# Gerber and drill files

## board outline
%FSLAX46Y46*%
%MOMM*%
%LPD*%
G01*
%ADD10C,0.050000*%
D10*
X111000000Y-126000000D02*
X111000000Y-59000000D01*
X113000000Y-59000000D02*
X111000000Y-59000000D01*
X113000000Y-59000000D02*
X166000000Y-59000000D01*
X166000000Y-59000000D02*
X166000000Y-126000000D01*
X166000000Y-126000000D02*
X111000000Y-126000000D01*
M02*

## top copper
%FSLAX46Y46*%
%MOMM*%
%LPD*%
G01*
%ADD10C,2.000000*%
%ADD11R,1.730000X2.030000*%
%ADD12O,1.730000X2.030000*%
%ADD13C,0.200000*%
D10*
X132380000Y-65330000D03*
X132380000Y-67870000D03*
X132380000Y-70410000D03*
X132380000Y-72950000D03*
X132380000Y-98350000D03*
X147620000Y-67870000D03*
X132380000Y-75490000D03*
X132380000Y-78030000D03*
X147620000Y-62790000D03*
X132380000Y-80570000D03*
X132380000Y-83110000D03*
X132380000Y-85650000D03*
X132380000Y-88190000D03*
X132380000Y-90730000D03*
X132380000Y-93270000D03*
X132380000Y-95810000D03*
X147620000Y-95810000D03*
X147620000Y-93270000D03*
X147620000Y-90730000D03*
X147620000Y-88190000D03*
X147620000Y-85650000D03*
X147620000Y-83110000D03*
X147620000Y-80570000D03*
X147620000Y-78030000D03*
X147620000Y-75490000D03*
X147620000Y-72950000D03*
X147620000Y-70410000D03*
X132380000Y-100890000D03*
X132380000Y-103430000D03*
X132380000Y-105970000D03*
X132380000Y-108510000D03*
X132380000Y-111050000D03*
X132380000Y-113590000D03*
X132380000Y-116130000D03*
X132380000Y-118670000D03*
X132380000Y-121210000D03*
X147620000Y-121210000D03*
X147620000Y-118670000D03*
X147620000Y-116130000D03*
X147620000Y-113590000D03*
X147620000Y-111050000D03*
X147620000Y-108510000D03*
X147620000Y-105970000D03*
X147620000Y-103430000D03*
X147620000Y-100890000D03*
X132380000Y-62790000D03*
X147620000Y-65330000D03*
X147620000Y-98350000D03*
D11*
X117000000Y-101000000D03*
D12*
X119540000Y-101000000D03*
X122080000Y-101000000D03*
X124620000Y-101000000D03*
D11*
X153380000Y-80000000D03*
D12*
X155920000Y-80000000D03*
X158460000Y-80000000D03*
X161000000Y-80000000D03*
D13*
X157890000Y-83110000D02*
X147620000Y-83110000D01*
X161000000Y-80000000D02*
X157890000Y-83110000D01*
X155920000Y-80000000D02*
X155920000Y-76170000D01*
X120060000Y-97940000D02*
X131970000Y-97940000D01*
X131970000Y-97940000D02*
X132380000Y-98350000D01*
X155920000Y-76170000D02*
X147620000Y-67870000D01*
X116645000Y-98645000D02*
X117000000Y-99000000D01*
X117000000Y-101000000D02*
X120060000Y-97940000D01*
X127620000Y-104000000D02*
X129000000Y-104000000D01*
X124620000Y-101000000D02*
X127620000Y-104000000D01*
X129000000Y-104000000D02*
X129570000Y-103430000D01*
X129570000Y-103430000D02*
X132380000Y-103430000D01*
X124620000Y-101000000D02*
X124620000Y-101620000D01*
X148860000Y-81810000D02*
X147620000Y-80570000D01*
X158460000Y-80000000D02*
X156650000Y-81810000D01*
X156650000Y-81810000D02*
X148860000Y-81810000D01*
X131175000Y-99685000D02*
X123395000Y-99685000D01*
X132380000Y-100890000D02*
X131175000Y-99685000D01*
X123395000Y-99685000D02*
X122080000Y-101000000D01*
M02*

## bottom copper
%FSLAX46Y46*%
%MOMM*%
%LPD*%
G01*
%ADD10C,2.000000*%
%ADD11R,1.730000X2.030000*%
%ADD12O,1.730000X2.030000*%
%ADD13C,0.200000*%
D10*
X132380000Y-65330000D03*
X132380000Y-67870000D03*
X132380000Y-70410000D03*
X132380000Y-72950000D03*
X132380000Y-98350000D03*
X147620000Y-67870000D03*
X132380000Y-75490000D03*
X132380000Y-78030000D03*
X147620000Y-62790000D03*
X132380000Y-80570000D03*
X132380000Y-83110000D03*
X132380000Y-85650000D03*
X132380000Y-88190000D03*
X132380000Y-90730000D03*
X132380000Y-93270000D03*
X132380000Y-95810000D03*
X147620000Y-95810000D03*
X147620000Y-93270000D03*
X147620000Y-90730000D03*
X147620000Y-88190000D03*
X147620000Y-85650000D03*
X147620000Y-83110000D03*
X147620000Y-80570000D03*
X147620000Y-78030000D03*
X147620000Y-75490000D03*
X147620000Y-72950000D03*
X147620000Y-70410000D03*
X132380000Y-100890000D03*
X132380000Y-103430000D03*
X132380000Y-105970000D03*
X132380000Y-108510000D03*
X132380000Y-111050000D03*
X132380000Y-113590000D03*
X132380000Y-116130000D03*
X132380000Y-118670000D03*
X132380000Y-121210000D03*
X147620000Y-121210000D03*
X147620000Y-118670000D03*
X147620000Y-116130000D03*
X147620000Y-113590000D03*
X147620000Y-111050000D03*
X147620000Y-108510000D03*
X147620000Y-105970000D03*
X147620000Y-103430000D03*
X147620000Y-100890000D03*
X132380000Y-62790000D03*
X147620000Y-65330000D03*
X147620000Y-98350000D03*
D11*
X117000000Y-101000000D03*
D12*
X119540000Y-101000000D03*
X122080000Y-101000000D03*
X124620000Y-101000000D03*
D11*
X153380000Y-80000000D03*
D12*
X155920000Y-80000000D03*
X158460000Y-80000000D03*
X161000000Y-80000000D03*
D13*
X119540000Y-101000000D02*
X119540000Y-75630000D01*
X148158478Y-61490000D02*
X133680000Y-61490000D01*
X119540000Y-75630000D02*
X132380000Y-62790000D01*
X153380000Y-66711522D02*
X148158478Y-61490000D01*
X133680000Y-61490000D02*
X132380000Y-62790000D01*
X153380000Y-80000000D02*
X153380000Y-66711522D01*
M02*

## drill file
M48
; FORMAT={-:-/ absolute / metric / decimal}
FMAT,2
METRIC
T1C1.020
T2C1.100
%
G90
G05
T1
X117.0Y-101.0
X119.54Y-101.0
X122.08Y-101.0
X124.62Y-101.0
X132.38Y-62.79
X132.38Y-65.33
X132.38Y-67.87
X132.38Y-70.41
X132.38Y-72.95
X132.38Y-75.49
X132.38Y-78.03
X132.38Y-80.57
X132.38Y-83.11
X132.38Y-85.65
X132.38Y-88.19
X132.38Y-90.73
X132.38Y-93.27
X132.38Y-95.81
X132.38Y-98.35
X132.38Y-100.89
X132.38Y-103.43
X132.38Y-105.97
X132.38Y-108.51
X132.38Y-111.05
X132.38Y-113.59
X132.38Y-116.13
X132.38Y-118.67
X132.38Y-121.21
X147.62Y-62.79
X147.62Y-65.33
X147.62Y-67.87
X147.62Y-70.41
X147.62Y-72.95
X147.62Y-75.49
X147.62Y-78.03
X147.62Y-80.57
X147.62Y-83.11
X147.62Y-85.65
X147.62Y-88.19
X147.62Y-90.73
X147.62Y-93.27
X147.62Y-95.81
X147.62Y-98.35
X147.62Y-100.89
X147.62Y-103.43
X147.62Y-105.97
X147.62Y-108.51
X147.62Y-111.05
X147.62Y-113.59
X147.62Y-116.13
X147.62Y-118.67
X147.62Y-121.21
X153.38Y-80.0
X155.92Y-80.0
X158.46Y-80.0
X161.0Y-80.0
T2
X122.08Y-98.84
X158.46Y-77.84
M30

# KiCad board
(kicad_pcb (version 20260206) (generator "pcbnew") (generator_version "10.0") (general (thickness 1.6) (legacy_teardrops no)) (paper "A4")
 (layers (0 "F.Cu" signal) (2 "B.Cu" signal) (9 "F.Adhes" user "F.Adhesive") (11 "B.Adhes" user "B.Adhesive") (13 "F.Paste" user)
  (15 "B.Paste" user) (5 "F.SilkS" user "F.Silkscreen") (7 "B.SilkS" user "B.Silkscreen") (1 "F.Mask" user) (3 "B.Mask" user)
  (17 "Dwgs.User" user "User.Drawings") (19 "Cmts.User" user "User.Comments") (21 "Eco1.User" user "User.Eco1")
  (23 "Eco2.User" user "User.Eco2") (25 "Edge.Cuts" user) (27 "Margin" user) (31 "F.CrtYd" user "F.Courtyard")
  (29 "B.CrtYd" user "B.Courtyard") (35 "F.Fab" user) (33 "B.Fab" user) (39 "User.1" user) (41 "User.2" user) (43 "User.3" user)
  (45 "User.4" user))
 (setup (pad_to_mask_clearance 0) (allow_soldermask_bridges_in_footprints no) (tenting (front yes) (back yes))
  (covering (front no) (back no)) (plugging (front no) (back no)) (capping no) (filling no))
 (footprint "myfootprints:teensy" (layer "F.Cu") (at 140 92)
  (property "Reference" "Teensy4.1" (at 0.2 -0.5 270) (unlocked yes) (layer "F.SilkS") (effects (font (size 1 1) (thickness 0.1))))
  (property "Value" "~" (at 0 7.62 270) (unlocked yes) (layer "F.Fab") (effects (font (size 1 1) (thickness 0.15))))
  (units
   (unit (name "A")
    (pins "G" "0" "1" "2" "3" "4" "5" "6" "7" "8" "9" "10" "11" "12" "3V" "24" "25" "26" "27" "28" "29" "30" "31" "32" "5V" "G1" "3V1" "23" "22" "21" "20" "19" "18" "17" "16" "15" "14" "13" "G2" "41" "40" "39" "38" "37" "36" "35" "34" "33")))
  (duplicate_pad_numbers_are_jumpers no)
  (pad "0" thru_hole circle (at -7.62 -26.67) (size 2 2) (drill 1.02) (layers "*.Cu" "*.Mask") (remove_unused_layers no)
   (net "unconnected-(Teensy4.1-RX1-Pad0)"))
  (pad "1" thru_hole circle (at -7.62 -24.13) (size 2 2) (drill 1.02) (layers "*.Cu" "*.Mask") (remove_unused_layers no)
   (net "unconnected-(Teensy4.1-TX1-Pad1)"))
  (pad "2" thru_hole circle (at -7.62 -21.59) (size 2 2) (drill 1.02) (layers "*.Cu" "*.Mask") (remove_unused_layers no)
   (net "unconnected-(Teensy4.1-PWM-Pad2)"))
  (pad "3" thru_hole circle (at -7.62 -19.05) (size 2 2) (drill 1.02) (layers "*.Cu" "*.Mask") (remove_unused_layers no)
   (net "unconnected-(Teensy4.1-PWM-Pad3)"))
  (pad "3V" thru_hole circle (at -7.62 6.35) (size 2 2) (drill 1.02) (layers "*.Cu" "*.Mask") (remove_unused_layers no) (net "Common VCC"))
  (pad "3V1" thru_hole circle (at 7.62 -24.13) (size 2 2) (drill 1.02) (layers "*.Cu" "*.Mask") (remove_unused_layers no) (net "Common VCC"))
  (pad "4" thru_hole circle (at -7.62 -16.51) (size 2 2) (drill 1.02) (layers "*.Cu" "*.Mask") (remove_unused_layers no)
   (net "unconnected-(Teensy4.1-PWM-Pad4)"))
  (pad "5" thru_hole circle (at -7.62 -13.97) (size 2 2) (drill 1.02) (layers "*.Cu" "*.Mask") (remove_unused_layers no)
   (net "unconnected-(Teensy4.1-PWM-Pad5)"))
  (pad "5V" thru_hole circle (at 7.62 -29.21) (size 2 2) (drill 1.02) (layers "*.Cu" "*.Mask") (remove_unused_layers no) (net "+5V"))
  (pad "6" thru_hole circle (at -7.62 -11.43) (size 2 2) (drill 1.02) (layers "*.Cu" "*.Mask") (remove_unused_layers no)
   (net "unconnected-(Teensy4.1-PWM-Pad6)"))
  (pad "7" thru_hole circle (at -7.62 -8.89) (size 2 2) (drill 1.02) (layers "*.Cu" "*.Mask") (remove_unused_layers no)
   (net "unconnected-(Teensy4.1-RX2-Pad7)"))
  (pad "8" thru_hole circle (at -7.62 -6.35) (size 2 2) (drill 1.02) (layers "*.Cu" "*.Mask") (remove_unused_layers no)
   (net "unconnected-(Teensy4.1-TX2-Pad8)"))
  (pad "9" thru_hole circle (at -7.62 -3.81) (size 2 2) (drill 1.02) (layers "*.Cu" "*.Mask") (remove_unused_layers no)
   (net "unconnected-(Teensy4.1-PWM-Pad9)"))
  (pad "10" thru_hole circle (at -7.62 -1.27) (size 2 2) (drill 1.02) (layers "*.Cu" "*.Mask") (remove_unused_layers no)
   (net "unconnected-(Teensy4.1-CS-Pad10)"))
  (pad "11" thru_hole circle (at -7.62 1.27) (size 2 2) (drill 1.02) (layers "*.Cu" "*.Mask") (remove_unused_layers no)
   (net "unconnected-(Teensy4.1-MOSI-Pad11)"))
  (pad "12" thru_hole circle (at -7.62 3.81) (size 2 2) (drill 1.02) (layers "*.Cu" "*.Mask") (remove_unused_layers no)
   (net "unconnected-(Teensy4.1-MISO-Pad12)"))
  (pad "13" thru_hole circle (at 7.62 3.81) (size 2 2) (drill 1.02) (layers "*.Cu" "*.Mask") (remove_unused_layers no)
   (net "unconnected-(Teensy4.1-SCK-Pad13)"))
  (pad "14" thru_hole circle (at 7.62 1.27) (size 2 2) (drill 1.02) (layers "*.Cu" "*.Mask") (remove_unused_layers no)
   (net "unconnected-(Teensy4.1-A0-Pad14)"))
  (pad "15" thru_hole circle (at 7.62 -1.27) (size 2 2) (drill 1.02) (layers "*.Cu" "*.Mask") (remove_unused_layers no)
   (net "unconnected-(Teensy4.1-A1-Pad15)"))
  (pad "16" thru_hole circle (at 7.62 -3.81) (size 2 2) (drill 1.02) (layers "*.Cu" "*.Mask") (remove_unused_layers no)
   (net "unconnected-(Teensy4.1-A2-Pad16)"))
  (pad "17" thru_hole circle (at 7.62 -6.35) (size 2 2) (drill 1.02) (layers "*.Cu" "*.Mask") (remove_unused_layers no)
   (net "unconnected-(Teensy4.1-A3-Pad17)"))
  (pad "18" thru_hole circle (at 7.62 -8.89) (size 2 2) (drill 1.02) (layers "*.Cu" "*.Mask") (remove_unused_layers no) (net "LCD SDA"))
  (pad "19" thru_hole circle (at 7.62 -11.43) (size 2 2) (drill 1.02) (layers "*.Cu" "*.Mask") (remove_unused_layers no) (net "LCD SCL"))
  (pad "20" thru_hole circle (at 7.62 -13.97) (size 2 2) (drill 1.02) (layers "*.Cu" "*.Mask") (remove_unused_layers no)
   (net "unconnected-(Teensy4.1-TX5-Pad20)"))
  (pad "21" thru_hole circle (at 7.62 -16.51) (size 2 2) (drill 1.02) (layers "*.Cu" "*.Mask") (remove_unused_layers no)
   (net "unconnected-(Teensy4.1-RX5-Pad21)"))
  (pad "22" thru_hole circle (at 7.62 -19.05) (size 2 2) (drill 1.02) (layers "*.Cu" "*.Mask") (remove_unused_layers no)
   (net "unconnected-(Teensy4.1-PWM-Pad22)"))
  (pad "23" thru_hole circle (at 7.62 -21.59) (size 2 2) (drill 1.02) (layers "*.Cu" "*.Mask") (remove_unused_layers no)
   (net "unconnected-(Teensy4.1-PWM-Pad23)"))
  (pad "24" thru_hole circle (at -7.62 8.89) (size 2 2) (drill 1.02) (layers "*.Cu" "*.Mask") (remove_unused_layers no) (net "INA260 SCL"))
  (pad "25" thru_hole circle (at -7.62 11.43) (size 2 2) (drill 1.02) (layers "*.Cu" "*.Mask") (remove_unused_layers no) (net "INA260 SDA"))
  (pad "26" thru_hole circle (at -7.62 13.97) (size 2 2) (drill 1.02) (layers "*.Cu" "*.Mask") (remove_unused_layers no)
   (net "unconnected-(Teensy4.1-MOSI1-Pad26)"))
  (pad "27" thru_hole circle (at -7.62 16.51) (size 2 2) (drill 1.02) (layers "*.Cu" "*.Mask") (remove_unused_layers no)
   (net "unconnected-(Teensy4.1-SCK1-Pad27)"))
  (pad "28" thru_hole circle (at -7.62 19.05) (size 2 2) (drill 1.02) (layers "*.Cu" "*.Mask") (remove_unused_layers no)
   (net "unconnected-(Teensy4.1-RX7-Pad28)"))
  (pad "29" thru_hole circle (at -7.62 21.59) (size 2 2) (drill 1.02) (layers "*.Cu" "*.Mask") (remove_unused_layers no)
   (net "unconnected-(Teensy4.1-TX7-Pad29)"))
  (pad "30" thru_hole circle (at -7.62 24.13) (size 2 2) (drill 1.02) (layers "*.Cu" "*.Mask") (remove_unused_layers no)
   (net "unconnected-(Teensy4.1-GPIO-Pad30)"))
  (pad "31" thru_hole circle (at -7.62 26.67) (size 2 2) (drill 1.02) (layers "*.Cu" "*.Mask") (remove_unused_layers no)
   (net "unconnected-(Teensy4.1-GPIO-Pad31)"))
  (pad "32" thru_hole circle (at -7.62 29.21) (size 2 2) (drill 1.02) (layers "*.Cu" "*.Mask") (remove_unused_layers no)
   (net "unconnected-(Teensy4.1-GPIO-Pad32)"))
  (pad "33" thru_hole circle (at 7.62 29.21) (size 2 2) (drill 1.02) (layers "*.Cu" "*.Mask") (remove_unused_layers no)
   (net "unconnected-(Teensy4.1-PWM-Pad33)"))
  (pad "34" thru_hole circle (at 7.62 26.67) (size 2 2) (drill 1.02) (layers "*.Cu" "*.Mask") (remove_unused_layers no)
   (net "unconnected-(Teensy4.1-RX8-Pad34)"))
  (pad "35" thru_hole circle (at 7.62 24.13) (size 2 2) (drill 1.02) (layers "*.Cu" "*.Mask") (remove_unused_layers no)
   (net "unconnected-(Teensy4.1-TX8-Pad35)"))
  (pad "36" thru_hole circle (at 7.62 21.59) (size 2 2) (drill 1.02) (layers "*.Cu" "*.Mask") (remove_unused_layers no)
   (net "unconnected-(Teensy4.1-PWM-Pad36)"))
  (pad "37" thru_hole circle (at 7.62 19.05) (size 2 2) (drill 1.02) (layers "*.Cu" "*.Mask") (remove_unused_layers no)
   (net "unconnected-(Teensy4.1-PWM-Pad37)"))
  (pad "38" thru_hole circle (at 7.62 16.51) (size 2 2) (drill 1.02) (layers "*.Cu" "*.Mask") (remove_unused_layers no)
   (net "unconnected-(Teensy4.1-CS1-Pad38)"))
  (pad "39" thru_hole circle (at 7.62 13.97) (size 2 2) (drill 1.02) (layers "*.Cu" "*.Mask") (remove_unused_layers no)
   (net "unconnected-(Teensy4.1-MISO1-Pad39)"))
  (pad "40" thru_hole circle (at 7.62 11.43) (size 2 2) (drill 1.02) (layers "*.Cu" "*.Mask") (remove_unused_layers no)
   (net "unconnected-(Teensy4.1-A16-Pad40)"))
  (pad "41" thru_hole circle (at 7.62 8.89) (size 2 2) (drill 1.02) (layers "*.Cu" "*.Mask") (remove_unused_layers no)
   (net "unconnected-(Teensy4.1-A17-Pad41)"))
  (pad "G" thru_hole circle (at -7.62 -29.21) (size 2 2) (drill 1.02) (layers "*.Cu" "*.Mask") (remove_unused_layers no) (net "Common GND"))
  (pad "G1" thru_hole circle (at 7.62 -26.67) (size 2 2) (drill 1.02) (layers "*.Cu" "*.Mask") (remove_unused_layers no)
   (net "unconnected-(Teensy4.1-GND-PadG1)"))
  (pad "G2" thru_hole circle (at 7.62 6.35) (size 2 2) (drill 1.02) (layers "*.Cu" "*.Mask") (remove_unused_layers no)
   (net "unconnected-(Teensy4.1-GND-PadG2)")))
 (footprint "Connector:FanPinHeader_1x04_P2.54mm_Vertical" (layer "F.Cu") (at 117 101)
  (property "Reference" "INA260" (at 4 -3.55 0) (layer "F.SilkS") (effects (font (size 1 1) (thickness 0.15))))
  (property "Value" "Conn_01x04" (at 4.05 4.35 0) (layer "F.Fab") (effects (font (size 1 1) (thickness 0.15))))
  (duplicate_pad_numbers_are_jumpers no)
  (pad "" np_thru_hole circle (at 5.08 -2.16 90) (size 1.1 1.1) (drill 1.1) (layers "*.Cu" "*.Mask"))
  (pad "1" thru_hole rect (at 0 0 90) (size 2.03 1.73) (drill 1.02) (layers "*.Cu" "*.Mask") (remove_unused_layers no) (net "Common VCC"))
  (pad "2" thru_hole oval (at 2.54 0 90) (size 2.03 1.73) (drill 1.02) (layers "*.Cu" "*.Mask") (remove_unused_layers no) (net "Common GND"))
  (pad "3" thru_hole oval (at 5.08 0 90) (size 2.03 1.73) (drill 1.02) (layers "*.Cu" "*.Mask") (remove_unused_layers no) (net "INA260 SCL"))
  (pad "4" thru_hole oval (at 7.62 0 90) (size 2.03 1.73) (drill 1.02) (layers "*.Cu" "*.Mask") (remove_unused_layers no) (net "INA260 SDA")))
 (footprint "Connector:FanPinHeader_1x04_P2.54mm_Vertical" (layer "F.Cu") (at 153.38 80)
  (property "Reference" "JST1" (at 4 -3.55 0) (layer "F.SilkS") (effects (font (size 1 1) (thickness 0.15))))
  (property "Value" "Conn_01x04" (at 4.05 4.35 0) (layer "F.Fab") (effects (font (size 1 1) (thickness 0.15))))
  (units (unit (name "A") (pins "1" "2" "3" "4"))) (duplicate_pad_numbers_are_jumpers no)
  (pad "" np_thru_hole circle (at 5.08 -2.16 90) (size 1.1 1.1) (drill 1.1) (layers "*.Cu" "*.Mask"))
  (pad "1" thru_hole rect (at 0 0 90) (size 2.03 1.73) (drill 1.02) (layers "*.Cu" "*.Mask") (remove_unused_layers no) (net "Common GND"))
  (pad "2" thru_hole oval (at 2.54 0 90) (size 2.03 1.73) (drill 1.02) (layers "*.Cu" "*.Mask") (remove_unused_layers no) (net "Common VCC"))
  (pad "3" thru_hole oval (at 5.08 0 90) (size 2.03 1.73) (drill 1.02) (layers "*.Cu" "*.Mask") (remove_unused_layers no) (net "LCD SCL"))
  (pad "4" thru_hole oval (at 7.62 0 90) (size 2.03 1.73) (drill 1.02) (layers "*.Cu" "*.Mask") (remove_unused_layers no) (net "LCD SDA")))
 (gr_line (start 111 126) (end 111 59) (stroke (width 0.05) (type default)) (layer "Edge.Cuts"))
 (gr_line (start 113 59) (end 111 59) (stroke (width 0.05) (type default)) (layer "Edge.Cuts"))
 (gr_line (start 113 59) (end 166 59) (stroke (width 0.05) (type default)) (layer "Edge.Cuts"))
 (gr_line (start 166 59) (end 166 126) (stroke (width 0.05) (type default)) (layer "Edge.Cuts"))
 (gr_line (start 166 126) (end 111 126) (stroke (width 0.05) (type default)) (layer "Edge.Cuts"))
 (segment (start 157.89 83.11) (end 147.62 83.11) (width 0.2) (layer "F.Cu") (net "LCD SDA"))
 (segment (start 161 80) (end 157.89 83.11) (width 0.2) (layer "F.Cu") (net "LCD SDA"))
 (segment (start 155.92 80) (end 155.92 76.17) (width 0.2) (layer "F.Cu") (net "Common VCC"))
 (segment (start 120.06 97.94) (end 131.97 97.94) (width 0.2) (layer "F.Cu") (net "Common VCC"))
 (segment (start 131.97 97.94) (end 132.38 98.35) (width 0.2) (layer "F.Cu") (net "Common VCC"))
 (segment (start 155.92 76.17) (end 147.62 67.87) (width 0.2) (layer "F.Cu") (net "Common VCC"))
 (segment (start 116.645 98.645) (end 117 99) (width 0.2) (layer "F.Cu") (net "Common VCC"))
 (segment (start 117 101) (end 120.06 97.94) (width 0.2) (layer "F.Cu") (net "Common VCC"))
 (segment (start 127.62 104) (end 129 104) (width 0.2) (layer "F.Cu") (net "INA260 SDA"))
 (segment (start 124.62 101) (end 127.62 104) (width 0.2) (layer "F.Cu") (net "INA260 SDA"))
 (segment (start 129 104) (end 129.57 103.43) (width 0.2) (layer "F.Cu") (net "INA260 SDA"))
 (segment (start 129.57 103.43) (end 132.38 103.43) (width 0.2) (layer "F.Cu") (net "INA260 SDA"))
 (segment (start 124.62 101) (end 124.62 101.62) (width 0.2) (layer "F.Cu") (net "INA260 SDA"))
 (segment (start 148.86 81.81) (end 147.62 80.57) (width 0.2) (layer "F.Cu") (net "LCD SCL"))
 (segment (start 158.46 80) (end 156.65 81.81) (width 0.2) (layer "F.Cu") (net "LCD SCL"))
 (segment (start 156.65 81.81) (end 148.86 81.81) (width 0.2) (layer "F.Cu") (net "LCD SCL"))
 (segment (start 131.175 99.685) (end 123.395 99.685) (width 0.2) (layer "F.Cu") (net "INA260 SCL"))
 (segment (start 132.38 100.89) (end 131.175 99.685) (width 0.2) (layer "F.Cu") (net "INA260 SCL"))
 (segment (start 123.395 99.685) (end 122.08 101) (width 0.2) (layer "F.Cu") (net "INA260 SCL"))
 (segment (start 119.54 101) (end 119.54 75.63) (width 0.2) (layer "B.Cu") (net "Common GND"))
 (segment (start 148.158478 61.49) (end 133.68 61.49) (width 0.2) (layer "B.Cu") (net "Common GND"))
 (segment (start 119.54 75.63) (end 132.38 62.79) (width 0.2) (layer "B.Cu") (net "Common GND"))
 (segment (start 153.38 66.711522) (end 148.158478 61.49) (width 0.2) (layer "B.Cu") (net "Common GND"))
 (segment (start 133.68 61.49) (end 132.38 62.79) (width 0.2) (layer "B.Cu") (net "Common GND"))
 (segment (start 153.38 80) (end 153.38 66.711522) (width 0.2) (layer "B.Cu") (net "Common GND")))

